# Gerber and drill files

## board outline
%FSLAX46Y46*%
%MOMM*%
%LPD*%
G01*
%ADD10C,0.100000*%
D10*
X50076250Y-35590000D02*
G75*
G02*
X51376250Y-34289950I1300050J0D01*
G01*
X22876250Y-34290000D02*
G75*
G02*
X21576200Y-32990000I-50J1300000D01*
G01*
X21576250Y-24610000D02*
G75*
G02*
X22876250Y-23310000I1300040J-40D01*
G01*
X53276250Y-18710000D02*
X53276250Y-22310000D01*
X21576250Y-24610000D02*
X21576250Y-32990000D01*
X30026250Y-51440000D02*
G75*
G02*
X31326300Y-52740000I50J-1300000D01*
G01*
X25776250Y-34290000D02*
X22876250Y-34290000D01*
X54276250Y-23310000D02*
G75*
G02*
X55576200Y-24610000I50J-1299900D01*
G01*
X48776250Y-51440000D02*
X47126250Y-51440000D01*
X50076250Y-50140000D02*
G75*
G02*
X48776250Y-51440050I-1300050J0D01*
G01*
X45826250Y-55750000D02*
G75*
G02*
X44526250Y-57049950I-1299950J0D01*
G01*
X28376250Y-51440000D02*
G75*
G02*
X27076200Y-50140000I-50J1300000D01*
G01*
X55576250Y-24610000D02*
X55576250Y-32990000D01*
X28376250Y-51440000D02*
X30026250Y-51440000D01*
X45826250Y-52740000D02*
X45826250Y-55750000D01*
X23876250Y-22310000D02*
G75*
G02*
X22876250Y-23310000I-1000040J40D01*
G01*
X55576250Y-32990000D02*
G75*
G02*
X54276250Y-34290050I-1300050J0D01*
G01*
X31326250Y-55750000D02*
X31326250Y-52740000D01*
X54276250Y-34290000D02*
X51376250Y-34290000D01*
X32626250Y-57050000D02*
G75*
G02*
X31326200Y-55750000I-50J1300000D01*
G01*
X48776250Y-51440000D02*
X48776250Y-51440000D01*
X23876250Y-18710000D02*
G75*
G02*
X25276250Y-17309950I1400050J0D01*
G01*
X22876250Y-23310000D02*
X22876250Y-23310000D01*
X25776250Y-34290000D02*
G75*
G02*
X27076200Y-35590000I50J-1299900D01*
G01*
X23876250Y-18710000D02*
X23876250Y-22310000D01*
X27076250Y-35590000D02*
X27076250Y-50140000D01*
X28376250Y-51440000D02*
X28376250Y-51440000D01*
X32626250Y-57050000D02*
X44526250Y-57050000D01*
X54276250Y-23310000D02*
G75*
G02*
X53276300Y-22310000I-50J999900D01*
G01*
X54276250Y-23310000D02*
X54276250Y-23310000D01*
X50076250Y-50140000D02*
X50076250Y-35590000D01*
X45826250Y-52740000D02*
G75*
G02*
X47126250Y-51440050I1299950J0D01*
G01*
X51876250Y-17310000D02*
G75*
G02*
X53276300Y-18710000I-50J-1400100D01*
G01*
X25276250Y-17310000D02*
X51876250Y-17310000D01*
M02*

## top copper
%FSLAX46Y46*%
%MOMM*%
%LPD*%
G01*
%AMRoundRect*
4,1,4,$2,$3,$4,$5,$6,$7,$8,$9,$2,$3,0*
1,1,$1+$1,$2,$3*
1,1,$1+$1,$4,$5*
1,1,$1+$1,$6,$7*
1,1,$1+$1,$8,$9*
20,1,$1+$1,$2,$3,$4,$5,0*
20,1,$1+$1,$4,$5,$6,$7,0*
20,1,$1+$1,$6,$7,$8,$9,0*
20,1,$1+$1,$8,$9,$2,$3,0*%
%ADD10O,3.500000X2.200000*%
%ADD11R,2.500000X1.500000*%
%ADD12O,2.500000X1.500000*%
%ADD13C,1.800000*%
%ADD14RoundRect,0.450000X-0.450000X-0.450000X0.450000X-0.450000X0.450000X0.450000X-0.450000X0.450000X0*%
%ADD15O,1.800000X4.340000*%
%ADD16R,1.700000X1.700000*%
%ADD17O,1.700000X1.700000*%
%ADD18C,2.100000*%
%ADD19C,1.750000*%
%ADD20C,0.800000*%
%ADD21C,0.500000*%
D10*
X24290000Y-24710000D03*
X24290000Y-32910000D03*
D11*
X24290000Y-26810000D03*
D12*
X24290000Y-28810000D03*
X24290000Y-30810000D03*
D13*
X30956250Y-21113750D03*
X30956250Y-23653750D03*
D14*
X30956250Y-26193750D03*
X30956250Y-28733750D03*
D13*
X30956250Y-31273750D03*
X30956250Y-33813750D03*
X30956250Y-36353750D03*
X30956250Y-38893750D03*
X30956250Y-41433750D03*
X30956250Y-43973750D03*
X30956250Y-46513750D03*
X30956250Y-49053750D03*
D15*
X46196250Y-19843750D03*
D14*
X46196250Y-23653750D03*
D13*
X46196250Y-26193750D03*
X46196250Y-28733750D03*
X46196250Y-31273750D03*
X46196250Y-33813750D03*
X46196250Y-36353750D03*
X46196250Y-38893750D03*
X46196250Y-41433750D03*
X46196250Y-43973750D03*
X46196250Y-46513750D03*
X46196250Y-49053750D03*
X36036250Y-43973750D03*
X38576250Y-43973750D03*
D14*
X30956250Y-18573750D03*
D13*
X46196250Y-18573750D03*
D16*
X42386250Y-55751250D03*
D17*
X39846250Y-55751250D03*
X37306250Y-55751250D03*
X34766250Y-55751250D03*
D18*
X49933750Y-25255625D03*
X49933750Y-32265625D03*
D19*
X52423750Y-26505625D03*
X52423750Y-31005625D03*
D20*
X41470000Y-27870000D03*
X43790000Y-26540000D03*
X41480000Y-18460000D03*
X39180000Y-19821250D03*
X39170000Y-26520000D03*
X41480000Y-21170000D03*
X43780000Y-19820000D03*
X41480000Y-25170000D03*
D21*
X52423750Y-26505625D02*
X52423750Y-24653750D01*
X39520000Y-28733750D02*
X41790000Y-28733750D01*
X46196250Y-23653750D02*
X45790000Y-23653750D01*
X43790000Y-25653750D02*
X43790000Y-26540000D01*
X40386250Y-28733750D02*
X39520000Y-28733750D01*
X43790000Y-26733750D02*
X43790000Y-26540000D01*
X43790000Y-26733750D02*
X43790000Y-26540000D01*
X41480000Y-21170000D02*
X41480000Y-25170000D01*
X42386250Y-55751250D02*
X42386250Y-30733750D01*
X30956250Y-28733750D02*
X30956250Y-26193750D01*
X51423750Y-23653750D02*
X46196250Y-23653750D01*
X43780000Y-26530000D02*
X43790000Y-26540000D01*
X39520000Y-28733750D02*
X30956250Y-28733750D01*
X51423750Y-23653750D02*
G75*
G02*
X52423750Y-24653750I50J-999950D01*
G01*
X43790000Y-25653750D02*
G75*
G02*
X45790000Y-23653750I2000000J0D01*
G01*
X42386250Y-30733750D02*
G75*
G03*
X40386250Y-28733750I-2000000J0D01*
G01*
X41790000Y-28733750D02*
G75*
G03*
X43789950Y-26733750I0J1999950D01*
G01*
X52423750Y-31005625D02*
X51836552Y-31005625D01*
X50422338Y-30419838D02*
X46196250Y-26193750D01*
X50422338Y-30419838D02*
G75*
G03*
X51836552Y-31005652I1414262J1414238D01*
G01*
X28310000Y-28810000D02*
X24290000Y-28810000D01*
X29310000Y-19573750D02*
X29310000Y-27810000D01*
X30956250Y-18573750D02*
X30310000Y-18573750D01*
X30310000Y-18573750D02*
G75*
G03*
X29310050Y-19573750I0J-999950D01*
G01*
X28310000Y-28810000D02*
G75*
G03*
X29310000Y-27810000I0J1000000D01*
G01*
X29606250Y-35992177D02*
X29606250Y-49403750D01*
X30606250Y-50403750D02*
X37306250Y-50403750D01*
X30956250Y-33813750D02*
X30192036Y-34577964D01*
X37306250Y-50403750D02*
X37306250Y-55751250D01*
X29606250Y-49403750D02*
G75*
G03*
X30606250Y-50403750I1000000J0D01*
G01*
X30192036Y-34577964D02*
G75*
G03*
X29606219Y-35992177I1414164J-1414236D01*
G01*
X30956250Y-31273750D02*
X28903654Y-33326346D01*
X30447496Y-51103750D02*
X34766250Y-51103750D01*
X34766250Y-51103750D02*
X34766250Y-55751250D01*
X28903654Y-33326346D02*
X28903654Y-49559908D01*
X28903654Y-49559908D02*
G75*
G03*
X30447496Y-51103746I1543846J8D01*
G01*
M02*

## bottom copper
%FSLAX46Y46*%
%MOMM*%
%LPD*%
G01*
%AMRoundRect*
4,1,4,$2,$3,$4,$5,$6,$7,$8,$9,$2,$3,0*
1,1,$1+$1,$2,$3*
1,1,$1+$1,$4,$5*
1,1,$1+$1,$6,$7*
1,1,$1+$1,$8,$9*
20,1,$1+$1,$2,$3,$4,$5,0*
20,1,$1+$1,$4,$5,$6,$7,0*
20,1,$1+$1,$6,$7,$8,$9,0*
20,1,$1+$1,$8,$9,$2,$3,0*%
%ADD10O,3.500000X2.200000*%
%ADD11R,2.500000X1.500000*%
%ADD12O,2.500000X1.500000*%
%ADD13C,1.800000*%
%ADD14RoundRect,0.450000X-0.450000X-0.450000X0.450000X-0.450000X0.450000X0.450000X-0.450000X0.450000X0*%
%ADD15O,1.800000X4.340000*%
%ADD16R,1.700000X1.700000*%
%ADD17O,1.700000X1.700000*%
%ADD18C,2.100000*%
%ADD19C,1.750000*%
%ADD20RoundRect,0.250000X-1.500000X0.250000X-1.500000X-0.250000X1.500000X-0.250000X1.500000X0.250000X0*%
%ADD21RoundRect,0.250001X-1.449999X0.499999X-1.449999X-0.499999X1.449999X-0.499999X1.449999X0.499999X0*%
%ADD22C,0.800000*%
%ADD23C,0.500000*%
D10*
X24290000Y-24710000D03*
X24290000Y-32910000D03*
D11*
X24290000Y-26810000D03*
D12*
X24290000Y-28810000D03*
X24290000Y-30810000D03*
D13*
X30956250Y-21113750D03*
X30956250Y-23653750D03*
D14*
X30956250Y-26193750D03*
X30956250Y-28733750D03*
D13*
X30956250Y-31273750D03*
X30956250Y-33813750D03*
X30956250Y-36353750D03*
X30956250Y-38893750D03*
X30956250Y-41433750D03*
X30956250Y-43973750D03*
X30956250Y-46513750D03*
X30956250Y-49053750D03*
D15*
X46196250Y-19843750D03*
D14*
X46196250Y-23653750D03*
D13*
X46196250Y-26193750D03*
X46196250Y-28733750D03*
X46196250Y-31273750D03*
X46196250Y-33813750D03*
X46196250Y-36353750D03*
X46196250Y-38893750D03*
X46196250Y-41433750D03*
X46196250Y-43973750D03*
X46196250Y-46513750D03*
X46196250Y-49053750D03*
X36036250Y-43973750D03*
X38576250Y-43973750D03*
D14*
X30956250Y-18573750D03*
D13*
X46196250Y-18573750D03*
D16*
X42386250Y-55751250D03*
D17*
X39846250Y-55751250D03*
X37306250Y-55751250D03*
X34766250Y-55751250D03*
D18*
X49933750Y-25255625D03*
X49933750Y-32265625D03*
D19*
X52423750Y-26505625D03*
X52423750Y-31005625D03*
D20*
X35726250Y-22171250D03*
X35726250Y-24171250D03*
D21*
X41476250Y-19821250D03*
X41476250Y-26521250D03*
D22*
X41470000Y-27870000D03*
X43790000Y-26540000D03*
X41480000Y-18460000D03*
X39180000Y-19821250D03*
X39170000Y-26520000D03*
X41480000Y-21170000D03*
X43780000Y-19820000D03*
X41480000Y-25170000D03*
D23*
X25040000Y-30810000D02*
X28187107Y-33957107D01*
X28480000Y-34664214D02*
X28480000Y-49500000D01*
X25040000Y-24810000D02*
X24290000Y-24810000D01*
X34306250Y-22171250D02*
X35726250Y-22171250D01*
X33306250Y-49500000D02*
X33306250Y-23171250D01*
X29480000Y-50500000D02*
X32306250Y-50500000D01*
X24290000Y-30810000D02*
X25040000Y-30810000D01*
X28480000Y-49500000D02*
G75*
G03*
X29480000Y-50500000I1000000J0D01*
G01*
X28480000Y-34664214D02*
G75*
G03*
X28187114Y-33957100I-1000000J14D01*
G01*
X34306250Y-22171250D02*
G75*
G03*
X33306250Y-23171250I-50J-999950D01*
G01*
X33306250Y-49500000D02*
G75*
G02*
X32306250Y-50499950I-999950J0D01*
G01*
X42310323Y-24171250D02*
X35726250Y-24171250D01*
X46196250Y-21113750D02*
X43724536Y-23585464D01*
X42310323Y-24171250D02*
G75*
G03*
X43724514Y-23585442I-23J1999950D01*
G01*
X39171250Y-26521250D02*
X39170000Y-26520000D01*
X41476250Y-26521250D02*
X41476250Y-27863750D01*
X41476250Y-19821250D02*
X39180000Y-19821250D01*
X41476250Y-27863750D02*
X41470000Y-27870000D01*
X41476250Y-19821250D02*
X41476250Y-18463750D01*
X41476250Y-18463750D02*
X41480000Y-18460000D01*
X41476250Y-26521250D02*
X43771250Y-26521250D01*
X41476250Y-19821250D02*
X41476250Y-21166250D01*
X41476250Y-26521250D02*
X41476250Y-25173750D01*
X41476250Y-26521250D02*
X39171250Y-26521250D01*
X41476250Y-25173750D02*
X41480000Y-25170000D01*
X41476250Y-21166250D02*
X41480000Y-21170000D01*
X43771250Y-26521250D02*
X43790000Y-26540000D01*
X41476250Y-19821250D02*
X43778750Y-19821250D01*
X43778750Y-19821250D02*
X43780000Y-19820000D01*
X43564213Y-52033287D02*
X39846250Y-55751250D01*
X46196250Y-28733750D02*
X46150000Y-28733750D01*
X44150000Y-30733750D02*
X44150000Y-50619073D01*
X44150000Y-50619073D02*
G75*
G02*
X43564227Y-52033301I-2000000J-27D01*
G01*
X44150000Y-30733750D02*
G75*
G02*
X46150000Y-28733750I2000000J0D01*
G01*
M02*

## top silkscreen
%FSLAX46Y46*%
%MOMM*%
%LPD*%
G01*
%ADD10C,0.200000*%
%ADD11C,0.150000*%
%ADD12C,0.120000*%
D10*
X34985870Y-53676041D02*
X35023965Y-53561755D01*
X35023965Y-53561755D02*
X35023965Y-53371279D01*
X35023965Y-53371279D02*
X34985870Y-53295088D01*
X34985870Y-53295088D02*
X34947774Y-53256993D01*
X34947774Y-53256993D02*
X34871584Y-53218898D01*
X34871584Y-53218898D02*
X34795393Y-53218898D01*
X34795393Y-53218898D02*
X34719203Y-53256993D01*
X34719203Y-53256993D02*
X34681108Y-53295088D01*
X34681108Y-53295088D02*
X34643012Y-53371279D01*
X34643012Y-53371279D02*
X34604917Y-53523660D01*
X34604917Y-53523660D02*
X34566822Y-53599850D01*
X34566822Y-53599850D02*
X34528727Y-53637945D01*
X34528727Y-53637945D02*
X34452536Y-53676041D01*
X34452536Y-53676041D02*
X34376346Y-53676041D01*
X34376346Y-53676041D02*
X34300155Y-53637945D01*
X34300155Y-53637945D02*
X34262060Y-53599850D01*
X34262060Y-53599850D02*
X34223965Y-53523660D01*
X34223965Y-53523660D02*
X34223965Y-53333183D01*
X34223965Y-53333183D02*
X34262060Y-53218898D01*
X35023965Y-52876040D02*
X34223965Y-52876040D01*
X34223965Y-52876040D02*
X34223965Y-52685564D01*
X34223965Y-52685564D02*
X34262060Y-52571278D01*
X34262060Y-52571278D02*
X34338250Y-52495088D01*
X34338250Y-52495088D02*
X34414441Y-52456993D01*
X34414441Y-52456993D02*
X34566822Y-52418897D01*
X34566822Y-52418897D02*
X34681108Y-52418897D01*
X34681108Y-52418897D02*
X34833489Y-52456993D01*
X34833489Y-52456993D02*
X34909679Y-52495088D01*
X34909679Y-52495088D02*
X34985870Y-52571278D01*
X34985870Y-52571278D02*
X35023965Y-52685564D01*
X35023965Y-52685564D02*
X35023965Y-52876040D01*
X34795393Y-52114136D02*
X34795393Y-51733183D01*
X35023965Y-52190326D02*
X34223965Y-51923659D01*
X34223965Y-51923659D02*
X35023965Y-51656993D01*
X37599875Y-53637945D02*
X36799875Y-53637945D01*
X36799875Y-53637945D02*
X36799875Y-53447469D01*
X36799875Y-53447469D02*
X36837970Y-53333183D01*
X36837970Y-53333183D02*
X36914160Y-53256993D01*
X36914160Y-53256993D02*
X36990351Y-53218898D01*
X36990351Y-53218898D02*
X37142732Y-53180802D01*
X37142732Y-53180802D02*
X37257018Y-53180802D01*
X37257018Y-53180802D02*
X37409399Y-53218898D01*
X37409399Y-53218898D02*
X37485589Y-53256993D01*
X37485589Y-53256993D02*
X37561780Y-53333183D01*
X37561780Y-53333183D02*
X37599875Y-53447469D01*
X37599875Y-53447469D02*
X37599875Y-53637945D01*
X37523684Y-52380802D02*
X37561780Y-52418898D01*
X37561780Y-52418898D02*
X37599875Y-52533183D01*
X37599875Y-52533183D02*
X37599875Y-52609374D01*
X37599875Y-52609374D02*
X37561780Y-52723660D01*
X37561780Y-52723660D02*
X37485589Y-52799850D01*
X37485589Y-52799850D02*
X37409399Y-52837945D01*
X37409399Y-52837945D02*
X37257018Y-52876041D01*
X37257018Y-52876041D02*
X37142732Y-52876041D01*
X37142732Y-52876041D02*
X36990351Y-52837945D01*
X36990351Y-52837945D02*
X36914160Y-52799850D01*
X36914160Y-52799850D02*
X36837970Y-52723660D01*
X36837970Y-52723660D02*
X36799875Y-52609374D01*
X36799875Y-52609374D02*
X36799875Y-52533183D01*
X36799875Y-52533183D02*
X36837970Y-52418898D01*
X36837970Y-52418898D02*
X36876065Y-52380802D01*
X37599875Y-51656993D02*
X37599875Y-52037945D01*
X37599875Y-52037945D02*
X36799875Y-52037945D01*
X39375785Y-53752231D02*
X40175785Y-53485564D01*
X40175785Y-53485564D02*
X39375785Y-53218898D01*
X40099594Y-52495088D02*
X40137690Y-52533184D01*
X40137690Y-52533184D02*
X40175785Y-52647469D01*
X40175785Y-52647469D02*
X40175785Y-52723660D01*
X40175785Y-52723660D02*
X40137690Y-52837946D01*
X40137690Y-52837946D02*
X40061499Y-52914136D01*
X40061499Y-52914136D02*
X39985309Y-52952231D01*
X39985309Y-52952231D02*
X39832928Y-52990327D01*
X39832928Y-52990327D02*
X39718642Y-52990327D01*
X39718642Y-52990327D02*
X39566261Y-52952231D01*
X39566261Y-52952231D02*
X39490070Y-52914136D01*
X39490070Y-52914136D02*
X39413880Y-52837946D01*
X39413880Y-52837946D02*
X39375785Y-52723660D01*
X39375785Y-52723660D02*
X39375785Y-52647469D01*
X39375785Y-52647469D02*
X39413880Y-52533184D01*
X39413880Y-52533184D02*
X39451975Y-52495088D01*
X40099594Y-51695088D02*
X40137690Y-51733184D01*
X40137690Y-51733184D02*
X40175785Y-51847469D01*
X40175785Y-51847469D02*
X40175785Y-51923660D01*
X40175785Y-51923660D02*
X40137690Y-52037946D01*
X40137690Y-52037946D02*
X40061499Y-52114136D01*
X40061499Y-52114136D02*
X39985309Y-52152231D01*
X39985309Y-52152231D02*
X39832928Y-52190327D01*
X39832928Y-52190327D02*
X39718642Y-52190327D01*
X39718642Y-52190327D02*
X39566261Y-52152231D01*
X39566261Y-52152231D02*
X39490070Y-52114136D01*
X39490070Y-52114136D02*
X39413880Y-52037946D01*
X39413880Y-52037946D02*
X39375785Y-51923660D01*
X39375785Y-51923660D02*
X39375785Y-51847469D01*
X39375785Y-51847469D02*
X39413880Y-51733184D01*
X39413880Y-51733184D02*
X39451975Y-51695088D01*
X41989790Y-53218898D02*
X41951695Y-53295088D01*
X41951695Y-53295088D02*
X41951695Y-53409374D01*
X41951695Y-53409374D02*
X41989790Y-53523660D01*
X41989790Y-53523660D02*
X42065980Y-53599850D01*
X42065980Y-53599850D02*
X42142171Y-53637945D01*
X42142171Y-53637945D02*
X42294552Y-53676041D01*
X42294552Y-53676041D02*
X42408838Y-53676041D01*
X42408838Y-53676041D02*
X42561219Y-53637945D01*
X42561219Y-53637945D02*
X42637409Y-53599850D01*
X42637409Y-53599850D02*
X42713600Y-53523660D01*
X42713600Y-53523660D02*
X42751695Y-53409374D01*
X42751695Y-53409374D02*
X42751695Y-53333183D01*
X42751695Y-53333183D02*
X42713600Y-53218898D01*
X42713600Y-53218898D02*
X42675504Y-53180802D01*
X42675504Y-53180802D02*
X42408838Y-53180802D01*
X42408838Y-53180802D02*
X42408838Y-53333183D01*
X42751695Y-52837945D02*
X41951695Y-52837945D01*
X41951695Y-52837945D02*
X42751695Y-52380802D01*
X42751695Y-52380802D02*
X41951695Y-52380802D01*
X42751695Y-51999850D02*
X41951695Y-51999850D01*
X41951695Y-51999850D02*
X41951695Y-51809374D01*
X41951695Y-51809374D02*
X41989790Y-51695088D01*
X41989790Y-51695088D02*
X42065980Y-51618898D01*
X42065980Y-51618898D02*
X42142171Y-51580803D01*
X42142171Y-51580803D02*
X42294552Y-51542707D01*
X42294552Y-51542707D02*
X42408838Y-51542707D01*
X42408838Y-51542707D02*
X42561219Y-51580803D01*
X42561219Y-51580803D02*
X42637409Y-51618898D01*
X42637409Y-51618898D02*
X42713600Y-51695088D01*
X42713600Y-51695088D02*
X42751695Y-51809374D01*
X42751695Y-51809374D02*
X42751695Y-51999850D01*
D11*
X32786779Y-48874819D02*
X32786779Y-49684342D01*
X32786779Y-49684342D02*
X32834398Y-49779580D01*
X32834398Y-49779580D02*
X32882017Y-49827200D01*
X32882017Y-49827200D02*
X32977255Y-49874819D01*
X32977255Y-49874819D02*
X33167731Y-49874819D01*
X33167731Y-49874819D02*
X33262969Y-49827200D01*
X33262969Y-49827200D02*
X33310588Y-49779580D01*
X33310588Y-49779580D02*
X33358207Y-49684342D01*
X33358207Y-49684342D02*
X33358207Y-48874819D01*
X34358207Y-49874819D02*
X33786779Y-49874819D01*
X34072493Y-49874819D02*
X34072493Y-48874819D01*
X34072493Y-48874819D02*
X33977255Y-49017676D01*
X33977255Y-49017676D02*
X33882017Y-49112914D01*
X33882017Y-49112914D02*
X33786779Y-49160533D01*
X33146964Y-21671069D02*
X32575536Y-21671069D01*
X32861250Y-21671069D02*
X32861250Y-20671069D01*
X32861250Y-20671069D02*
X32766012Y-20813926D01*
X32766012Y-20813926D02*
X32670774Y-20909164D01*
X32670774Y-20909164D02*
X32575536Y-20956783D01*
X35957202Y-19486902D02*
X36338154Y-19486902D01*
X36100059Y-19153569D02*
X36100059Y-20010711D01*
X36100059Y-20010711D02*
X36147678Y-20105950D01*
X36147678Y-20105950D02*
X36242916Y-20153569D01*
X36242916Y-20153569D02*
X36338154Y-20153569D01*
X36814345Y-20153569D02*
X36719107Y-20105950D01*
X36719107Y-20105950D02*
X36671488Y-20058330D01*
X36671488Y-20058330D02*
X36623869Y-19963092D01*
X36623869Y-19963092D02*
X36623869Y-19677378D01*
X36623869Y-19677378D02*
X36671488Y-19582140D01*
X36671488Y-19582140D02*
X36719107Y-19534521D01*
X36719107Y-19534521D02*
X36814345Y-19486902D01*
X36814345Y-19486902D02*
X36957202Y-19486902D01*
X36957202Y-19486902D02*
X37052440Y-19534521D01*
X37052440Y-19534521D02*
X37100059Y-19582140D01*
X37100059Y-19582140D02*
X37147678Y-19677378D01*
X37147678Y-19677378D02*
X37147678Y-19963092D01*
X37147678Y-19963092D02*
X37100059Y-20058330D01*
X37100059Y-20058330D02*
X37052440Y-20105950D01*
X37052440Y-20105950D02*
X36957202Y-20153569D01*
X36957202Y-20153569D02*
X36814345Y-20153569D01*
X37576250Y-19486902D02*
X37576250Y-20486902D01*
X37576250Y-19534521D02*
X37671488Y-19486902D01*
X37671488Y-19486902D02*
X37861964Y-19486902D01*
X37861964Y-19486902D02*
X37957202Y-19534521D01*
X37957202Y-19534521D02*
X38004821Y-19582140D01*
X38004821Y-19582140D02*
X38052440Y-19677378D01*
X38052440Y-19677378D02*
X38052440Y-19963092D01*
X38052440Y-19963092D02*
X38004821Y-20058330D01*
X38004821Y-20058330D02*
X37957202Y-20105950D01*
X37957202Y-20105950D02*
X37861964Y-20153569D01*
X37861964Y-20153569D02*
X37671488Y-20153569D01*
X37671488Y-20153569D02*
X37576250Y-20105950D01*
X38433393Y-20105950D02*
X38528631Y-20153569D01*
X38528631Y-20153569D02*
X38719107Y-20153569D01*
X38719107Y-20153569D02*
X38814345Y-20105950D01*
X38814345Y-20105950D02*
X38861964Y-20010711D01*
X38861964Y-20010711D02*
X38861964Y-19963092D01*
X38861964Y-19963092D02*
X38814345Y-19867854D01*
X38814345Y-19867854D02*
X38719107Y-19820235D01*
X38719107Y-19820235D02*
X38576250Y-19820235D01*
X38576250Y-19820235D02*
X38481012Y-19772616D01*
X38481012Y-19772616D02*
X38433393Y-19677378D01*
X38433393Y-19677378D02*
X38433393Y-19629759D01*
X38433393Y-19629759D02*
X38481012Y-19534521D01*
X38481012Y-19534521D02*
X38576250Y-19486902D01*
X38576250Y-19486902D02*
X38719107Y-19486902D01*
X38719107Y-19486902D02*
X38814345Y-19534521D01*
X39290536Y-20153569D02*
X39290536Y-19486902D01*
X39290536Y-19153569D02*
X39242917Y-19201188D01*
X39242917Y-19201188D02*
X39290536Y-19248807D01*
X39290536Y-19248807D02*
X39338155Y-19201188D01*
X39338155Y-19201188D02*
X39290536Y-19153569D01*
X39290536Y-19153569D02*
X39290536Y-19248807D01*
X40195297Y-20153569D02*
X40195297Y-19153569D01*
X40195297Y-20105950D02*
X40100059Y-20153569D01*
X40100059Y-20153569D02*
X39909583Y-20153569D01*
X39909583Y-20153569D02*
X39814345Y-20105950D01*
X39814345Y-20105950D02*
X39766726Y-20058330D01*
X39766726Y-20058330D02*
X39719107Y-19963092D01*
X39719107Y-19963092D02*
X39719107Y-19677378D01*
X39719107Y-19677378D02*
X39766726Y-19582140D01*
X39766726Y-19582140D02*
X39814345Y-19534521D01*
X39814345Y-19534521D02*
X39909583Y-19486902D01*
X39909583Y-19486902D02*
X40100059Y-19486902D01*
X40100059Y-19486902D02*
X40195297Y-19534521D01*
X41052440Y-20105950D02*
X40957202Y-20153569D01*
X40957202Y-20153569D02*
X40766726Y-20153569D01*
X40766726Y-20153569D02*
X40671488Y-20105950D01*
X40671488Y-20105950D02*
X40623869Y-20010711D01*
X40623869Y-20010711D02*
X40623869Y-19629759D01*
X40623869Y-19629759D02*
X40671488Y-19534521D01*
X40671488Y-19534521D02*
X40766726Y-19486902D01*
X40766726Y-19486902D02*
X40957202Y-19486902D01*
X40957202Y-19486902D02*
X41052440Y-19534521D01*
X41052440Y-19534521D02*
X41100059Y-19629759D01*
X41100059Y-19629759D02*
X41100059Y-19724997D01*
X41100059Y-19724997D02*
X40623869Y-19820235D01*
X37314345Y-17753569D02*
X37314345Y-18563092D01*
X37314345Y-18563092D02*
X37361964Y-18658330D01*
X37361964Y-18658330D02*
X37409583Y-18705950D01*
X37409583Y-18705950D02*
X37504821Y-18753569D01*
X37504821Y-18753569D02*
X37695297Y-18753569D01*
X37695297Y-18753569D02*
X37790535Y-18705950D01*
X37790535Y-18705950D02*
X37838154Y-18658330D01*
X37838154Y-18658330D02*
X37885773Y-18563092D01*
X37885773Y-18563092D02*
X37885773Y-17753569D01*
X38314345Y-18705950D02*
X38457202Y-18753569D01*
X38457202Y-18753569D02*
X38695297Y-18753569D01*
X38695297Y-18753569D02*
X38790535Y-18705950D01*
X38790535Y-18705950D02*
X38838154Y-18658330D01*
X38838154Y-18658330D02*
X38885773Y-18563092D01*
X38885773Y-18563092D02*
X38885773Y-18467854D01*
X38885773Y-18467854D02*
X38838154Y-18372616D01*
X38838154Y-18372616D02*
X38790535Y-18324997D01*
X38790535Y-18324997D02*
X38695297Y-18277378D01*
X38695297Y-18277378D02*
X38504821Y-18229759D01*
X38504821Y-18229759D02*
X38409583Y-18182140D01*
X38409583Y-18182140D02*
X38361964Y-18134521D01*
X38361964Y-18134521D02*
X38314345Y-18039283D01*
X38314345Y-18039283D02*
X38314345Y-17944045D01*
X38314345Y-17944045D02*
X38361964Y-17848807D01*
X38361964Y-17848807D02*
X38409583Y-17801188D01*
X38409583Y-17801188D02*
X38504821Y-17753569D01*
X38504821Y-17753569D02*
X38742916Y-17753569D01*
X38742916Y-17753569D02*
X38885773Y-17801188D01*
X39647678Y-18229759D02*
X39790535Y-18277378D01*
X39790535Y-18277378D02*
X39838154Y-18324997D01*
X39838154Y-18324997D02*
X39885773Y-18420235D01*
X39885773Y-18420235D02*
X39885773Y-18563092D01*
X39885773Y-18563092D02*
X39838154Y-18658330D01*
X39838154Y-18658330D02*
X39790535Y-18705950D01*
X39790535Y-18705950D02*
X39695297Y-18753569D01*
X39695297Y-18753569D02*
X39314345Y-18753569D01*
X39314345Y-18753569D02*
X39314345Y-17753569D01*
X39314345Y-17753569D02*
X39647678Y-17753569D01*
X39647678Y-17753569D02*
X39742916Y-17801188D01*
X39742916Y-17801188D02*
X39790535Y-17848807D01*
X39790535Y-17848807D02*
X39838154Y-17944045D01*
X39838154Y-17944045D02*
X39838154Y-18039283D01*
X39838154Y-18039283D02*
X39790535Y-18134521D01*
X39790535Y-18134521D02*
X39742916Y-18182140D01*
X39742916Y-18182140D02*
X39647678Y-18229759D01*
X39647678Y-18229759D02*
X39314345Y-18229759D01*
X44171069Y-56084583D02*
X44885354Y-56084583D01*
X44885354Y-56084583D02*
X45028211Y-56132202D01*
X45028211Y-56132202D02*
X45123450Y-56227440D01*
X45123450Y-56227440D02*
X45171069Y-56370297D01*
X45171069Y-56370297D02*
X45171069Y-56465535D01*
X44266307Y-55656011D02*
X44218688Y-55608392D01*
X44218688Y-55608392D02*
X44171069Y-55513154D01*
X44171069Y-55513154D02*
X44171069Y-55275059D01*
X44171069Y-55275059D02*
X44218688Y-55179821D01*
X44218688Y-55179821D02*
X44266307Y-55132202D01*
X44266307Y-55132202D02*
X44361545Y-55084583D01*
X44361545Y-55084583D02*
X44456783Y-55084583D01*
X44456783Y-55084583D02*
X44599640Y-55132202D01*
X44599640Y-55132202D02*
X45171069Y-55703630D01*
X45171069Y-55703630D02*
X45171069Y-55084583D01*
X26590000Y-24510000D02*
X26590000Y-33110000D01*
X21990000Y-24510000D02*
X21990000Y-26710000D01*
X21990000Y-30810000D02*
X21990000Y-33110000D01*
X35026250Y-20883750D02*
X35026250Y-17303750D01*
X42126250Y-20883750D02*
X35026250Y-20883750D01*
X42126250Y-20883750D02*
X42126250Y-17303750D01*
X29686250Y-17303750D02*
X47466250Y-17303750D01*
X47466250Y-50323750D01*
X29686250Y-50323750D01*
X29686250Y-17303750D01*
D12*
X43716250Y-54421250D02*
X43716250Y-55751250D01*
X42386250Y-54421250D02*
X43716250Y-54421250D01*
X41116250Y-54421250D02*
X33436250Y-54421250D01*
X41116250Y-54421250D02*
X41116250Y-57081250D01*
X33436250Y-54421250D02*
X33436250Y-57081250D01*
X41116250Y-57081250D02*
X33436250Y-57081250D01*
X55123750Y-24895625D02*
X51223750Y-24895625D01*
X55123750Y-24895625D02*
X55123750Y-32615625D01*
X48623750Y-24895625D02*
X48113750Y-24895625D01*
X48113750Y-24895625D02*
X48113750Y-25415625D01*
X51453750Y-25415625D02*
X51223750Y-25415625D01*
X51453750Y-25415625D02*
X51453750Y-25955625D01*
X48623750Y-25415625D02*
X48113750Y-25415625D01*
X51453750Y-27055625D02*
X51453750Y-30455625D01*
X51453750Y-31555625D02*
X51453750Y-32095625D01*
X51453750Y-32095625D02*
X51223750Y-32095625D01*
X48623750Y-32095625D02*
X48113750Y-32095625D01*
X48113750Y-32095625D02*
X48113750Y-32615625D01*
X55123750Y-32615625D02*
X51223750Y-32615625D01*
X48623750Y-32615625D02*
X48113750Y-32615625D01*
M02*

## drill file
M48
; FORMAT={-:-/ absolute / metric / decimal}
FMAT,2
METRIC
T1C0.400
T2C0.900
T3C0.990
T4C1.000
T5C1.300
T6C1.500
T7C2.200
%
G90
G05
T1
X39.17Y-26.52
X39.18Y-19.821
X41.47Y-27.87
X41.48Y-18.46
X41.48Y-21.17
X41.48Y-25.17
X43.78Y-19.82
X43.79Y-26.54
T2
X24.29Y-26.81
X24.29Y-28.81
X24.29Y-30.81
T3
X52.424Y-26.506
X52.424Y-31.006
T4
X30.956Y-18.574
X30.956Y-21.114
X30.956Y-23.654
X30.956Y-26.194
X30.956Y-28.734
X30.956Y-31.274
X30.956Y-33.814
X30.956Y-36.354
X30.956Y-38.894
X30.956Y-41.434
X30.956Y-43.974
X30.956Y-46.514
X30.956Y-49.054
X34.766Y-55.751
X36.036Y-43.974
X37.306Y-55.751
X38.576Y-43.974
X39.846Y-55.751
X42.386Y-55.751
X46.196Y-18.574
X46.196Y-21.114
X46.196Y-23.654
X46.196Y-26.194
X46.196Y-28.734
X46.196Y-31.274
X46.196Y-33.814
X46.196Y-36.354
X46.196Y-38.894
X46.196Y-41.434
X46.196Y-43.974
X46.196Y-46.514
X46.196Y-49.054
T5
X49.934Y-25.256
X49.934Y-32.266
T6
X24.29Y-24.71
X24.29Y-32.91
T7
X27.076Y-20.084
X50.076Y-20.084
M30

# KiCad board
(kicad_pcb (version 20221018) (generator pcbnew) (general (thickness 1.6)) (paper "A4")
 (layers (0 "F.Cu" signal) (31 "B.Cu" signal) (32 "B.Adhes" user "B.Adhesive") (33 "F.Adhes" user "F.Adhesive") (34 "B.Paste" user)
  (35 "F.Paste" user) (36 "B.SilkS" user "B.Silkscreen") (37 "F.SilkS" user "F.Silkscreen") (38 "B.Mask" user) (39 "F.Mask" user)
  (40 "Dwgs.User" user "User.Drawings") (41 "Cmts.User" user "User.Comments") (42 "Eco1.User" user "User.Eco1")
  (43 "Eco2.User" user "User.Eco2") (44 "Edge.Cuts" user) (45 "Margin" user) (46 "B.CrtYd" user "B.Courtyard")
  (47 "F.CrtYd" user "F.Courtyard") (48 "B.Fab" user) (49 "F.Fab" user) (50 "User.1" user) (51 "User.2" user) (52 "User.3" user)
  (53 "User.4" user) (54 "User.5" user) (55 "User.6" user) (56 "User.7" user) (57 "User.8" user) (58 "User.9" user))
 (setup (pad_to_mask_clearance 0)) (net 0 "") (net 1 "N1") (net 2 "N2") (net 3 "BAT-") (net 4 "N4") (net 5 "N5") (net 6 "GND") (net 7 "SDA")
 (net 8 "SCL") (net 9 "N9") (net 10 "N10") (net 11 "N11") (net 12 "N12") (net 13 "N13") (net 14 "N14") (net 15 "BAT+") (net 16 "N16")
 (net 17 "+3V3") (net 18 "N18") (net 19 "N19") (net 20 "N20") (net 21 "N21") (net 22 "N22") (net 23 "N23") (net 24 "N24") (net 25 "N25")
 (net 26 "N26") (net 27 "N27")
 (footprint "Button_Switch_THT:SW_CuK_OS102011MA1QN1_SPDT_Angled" (layer "F.Cu") (at 24.29 26.81 -90)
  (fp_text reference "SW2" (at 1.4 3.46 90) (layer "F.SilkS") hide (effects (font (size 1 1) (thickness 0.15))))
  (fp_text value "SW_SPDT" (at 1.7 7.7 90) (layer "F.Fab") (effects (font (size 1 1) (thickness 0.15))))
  (fp_line (start -2.3 -2.3) (end 6.3 -2.3) (stroke (width 0.15) (type solid)) (layer "F.SilkS"))
  (fp_line (start -2.3 2.3) (end -0.1 2.3) (stroke (width 0.15) (type solid)) (layer "F.SilkS"))
  (fp_line (start 4 2.3) (end 6.3 2.3) (stroke (width 0.15) (type solid)) (layer "F.SilkS"))
  (pad "" thru_hole oval (at -2.1 0 270) (size 2.2 3.5) (drill 1.5) (layers "*.Cu" "*.Mask"))
  (pad "" thru_hole oval (at 6.1 0 270) (size 2.2 3.5) (drill 1.5) (layers "*.Cu" "*.Mask"))
  (pad "1" thru_hole rect (at 0 0 270) (size 1.5 2.5) (drill 0.9) (layers "*.Cu" "*.Mask") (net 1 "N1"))
  (pad "2" thru_hole oval (at 2 0 270) (size 1.5 2.5) (drill 0.9) (layers "*.Cu" "*.Mask") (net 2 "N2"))
  (pad "3" thru_hole oval (at 4 0 270) (size 1.5 2.5) (drill 0.9) (layers "*.Cu" "*.Mask") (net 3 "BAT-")))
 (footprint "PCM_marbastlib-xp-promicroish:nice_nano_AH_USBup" (layer "F.Cu") (at 38.57625 35.08375)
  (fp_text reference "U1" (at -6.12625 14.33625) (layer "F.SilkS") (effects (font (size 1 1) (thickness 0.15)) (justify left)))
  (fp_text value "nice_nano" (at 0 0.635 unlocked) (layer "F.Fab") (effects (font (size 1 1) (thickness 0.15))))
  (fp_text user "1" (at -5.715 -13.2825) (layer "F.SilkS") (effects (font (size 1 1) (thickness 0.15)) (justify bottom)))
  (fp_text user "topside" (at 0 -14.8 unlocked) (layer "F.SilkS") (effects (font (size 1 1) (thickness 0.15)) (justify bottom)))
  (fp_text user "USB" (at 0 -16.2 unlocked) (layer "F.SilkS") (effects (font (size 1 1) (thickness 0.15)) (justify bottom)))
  (fp_line (start -3.55 -14.2) (end -3.55 -17.78) (stroke (width 0.15) (type default)) (layer "F.SilkS"))
  (fp_line (start 3.55 -14.2) (end -3.55 -14.2) (stroke (width 0.15) (type default)) (layer "F.SilkS"))
  (fp_line (start 3.55 -14.2) (end 3.55 -17.78) (stroke (width 0.15) (type default)) (layer "F.SilkS"))
  (fp_rect (start -8.89 -17.78) (end 8.89 15.24) (stroke (width 0.15) (type solid)) (fill none) (layer "F.SilkS"))
  (pad "1" thru_hole circle (at -7.62 -13.97) (size 1.8 1.8) (drill 1) (layers "*.Cu" "B.Mask") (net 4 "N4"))
  (pad "2" thru_hole circle (at -7.62 -11.43) (size 1.8 1.8) (drill 1) (layers "*.Cu" "B.Mask") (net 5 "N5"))
  (pad "3" thru_hole roundrect (at -7.62 -8.89) (size 1.8 1.8) (drill 1) (layers "*.Cu" "B.Mask") (roundrect_rratio 0.25) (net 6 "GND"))
  (pad "4" thru_hole roundrect (at -7.62 -6.35) (size 1.8 1.8) (drill 1) (layers "*.Cu" "B.Mask") (roundrect_rratio 0.25) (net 6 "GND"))
  (pad "5" thru_hole circle (at -7.62 -3.81) (size 1.8 1.8) (drill 1) (layers "*.Cu" "B.Mask") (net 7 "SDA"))
  (pad "6" thru_hole circle (at -7.62 -1.27) (size 1.8 1.8) (drill 1) (layers "*.Cu" "B.Mask") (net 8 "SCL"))
  (pad "7" thru_hole circle (at -7.62 1.27) (size 1.8 1.8) (drill 1) (layers "*.Cu" "B.Mask") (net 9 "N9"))
  (pad "8" thru_hole circle (at -7.62 3.81) (size 1.8 1.8) (drill 1) (layers "*.Cu" "B.Mask") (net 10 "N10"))
  (pad "9" thru_hole circle (at -7.62 6.35) (size 1.8 1.8) (drill 1) (layers "*.Cu" "B.Mask") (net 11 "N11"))
  (pad "10" thru_hole circle (at -7.62 8.89) (size 1.8 1.8) (drill 1) (layers "*.Cu" "B.Mask") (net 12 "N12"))
  (pad "11" thru_hole circle (at -7.62 11.43) (size 1.8 1.8) (drill 1) (layers "*.Cu" "B.Mask") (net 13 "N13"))
  (pad "12" thru_hole circle (at -7.62 13.97) (size 1.8 1.8) (drill 1) (layers "*.Cu" "B.Mask") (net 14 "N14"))
  (pad "13" thru_hole oval (at 7.62 -13.97) (size 1.8 4.34) (drill 1 (offset 0 -1.27)) (layers "*.Cu" "B.Mask") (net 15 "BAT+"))
  (pad "14" thru_hole roundrect (at 7.62 -11.43) (size 1.8 1.8) (drill 1) (layers "*.Cu" "B.Mask") (roundrect_rratio 0.25) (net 6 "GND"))
  (pad "15" thru_hole circle (at 7.62 -8.89) (size 1.8 1.8) (drill 1) (layers "*.Cu" "B.Mask") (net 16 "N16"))
  (pad "16" thru_hole circle (at 7.62 -6.35) (size 1.8 1.8) (drill 1) (layers "*.Cu" "B.Mask") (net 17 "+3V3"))
  (pad "17" thru_hole circle (at 7.62 -3.81) (size 1.8 1.8) (drill 1) (layers "*.Cu" "B.Mask") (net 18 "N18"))
  (pad "18" thru_hole circle (at 7.62 -1.27) (size 1.8 1.8) (drill 1) (layers "*.Cu" "B.Mask") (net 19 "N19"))
  (pad "19" thru_hole circle (at 7.62 1.27) (size 1.8 1.8) (drill 1) (layers "*.Cu" "B.Mask") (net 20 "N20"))
  (pad "20" thru_hole circle (at 7.62 3.81) (size 1.8 1.8) (drill 1) (layers "*.Cu" "B.Mask") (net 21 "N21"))
  (pad "21" thru_hole circle (at 7.62 6.35) (size 1.8 1.8) (drill 1) (layers "*.Cu" "B.Mask") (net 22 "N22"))
  (pad "22" thru_hole circle (at 7.62 8.89) (size 1.8 1.8) (drill 1) (layers "*.Cu" "B.Mask") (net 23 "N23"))
  (pad "23" thru_hole circle (at 7.62 11.43) (size 1.8 1.8) (drill 1) (layers "*.Cu" "B.Mask") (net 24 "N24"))
  (pad "24" thru_hole circle (at 7.62 13.97) (size 1.8 1.8) (drill 1) (layers "*.Cu" "B.Mask") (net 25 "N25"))
  (pad "26" thru_hole circle (at -2.54 8.89) (size 1.8 1.8) (drill 1) (layers "*.Cu" "B.Mask") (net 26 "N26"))
  (pad "27" thru_hole circle (at 0 8.89) (size 1.8 1.8) (drill 1) (layers "*.Cu" "B.Mask") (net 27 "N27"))
  (pad "28" thru_hole roundrect (at -7.62 -16.51) (size 1.8 1.8) (drill 1) (layers "*.Cu" "B.Mask") (roundrect_rratio 0.25) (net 2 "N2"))
  (pad "29" thru_hole circle (at 7.62 -16.51) (size 1.8 1.8) (drill 1) (layers "*.Cu" "B.Mask") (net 15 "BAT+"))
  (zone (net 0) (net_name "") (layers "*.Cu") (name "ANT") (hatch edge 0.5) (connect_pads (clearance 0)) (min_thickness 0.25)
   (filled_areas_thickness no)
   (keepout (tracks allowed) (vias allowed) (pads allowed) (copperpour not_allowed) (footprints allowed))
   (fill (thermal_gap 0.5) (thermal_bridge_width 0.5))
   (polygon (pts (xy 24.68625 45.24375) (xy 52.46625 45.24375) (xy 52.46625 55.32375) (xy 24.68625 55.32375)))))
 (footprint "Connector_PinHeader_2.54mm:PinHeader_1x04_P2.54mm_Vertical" (layer "F.Cu") (at 42.38625 55.75125 -90)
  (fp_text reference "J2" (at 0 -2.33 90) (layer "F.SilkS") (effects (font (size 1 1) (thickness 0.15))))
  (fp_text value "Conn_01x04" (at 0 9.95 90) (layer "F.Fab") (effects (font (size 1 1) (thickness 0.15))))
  (fp_line (start -1.33 -1.33) (end 0 -1.33) (stroke (width 0.12) (type solid)) (layer "F.SilkS"))
  (fp_line (start -1.33 0) (end -1.33 -1.33) (stroke (width 0.12) (type solid)) (layer "F.SilkS"))
  (fp_line (start -1.33 1.27) (end -1.33 8.95) (stroke (width 0.12) (type solid)) (layer "F.SilkS"))
  (fp_line (start -1.33 1.27) (end 1.33 1.27) (stroke (width 0.12) (type solid)) (layer "F.SilkS"))
  (fp_line (start -1.33 8.95) (end 1.33 8.95) (stroke (width 0.12) (type solid)) (layer "F.SilkS"))
  (fp_line (start 1.33 1.27) (end 1.33 8.95) (stroke (width 0.12) (type solid)) (layer "F.SilkS"))
  (pad "1" thru_hole rect (at 0 0 270) (size 1.7 1.7) (drill 1) (layers "*.Cu" "*.Mask") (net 6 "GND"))
  (pad "2" thru_hole oval (at 0 2.54 270) (size 1.7 1.7) (drill 1) (layers "*.Cu" "*.Mask") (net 17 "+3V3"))
  (pad "3" thru_hole oval (at 0 5.08 270) (size 1.7 1.7) (drill 1) (layers "*.Cu" "*.Mask") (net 8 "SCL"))
  (pad "4" thru_hole oval (at 0 7.62 270) (size 1.7 1.7) (drill 1) (layers "*.Cu" "*.Mask") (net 7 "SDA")))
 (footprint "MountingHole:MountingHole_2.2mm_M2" (layer "F.Cu") (at 50.07625 20.08375)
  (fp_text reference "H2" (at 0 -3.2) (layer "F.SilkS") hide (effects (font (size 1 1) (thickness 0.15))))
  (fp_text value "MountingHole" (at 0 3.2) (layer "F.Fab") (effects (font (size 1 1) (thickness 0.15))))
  (pad "" np_thru_hole circle (at 0 0) (size 2.2 2.2) (drill 2.2) (layers "*.Cu" "*.Mask")))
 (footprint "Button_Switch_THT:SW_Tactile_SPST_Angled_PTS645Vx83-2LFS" (layer "F.Cu") (at 52.42375 26.505625 -90)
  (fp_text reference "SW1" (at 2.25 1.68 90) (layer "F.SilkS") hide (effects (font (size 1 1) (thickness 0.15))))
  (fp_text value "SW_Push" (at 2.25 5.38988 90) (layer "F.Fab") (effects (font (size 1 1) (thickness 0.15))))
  (fp_line (start -1.61 -2.7) (end -1.61 1.2) (stroke (width 0.12) (type solid)) (layer "F.SilkS"))
  (fp_line (start -1.61 -2.7) (end 6.11 -2.7) (stroke (width 0.12) (type solid)) (layer "F.SilkS"))
  (fp_line (start -1.61 3.8) (end -1.61 4.31) (stroke (width 0.12) (type solid)) (layer "F.SilkS"))
  (fp_line (start -1.61 4.31) (end -1.09 4.31) (stroke (width 0.12) (type solid)) (layer "F.SilkS"))
  (fp_line (start -1.09 0.97) (end -1.09 1.2) (stroke (width 0.12) (type solid)) (layer "F.SilkS"))
  (fp_line (start -1.09 0.97) (end -0.55 0.97) (stroke (width 0.12) (type solid)) (layer "F.SilkS"))
  (fp_line (start -1.09 3.8) (end -1.09 4.31) (stroke (width 0.12) (type solid)) (layer "F.SilkS"))
  (fp_line (start 0.55 0.97) (end 3.95 0.97) (stroke (width 0.12) (type solid)) (layer "F.SilkS"))
  (fp_line (start 5.05 0.97) (end 5.59 0.97) (stroke (width 0.12) (type solid)) (layer "F.SilkS"))
  (fp_line (start 5.59 0.97) (end 5.59 1.2) (stroke (width 0.12) (type solid)) (layer "F.SilkS"))
  (fp_line (start 5.59 3.8) (end 5.59 4.31) (stroke (width 0.12) (type solid)) (layer "F.SilkS"))
  (fp_line (start 5.59 4.31) (end 6.11 4.31) (stroke (width 0.12) (type solid)) (layer "F.SilkS"))
  (fp_line (start 6.11 -2.7) (end 6.11 1.2) (stroke (width 0.12) (type solid)) (layer "F.SilkS"))
  (fp_line (start 6.11 3.8) (end 6.11 4.31) (stroke (width 0.12) (type solid)) (layer "F.SilkS"))
  (pad "" thru_hole circle (at -1.25 2.49 270) (size 2.1 2.1) (drill 1.3) (layers "*.Cu" "*.Mask"))
  (pad "" thru_hole circle (at 5.76 2.49 270) (size 2.1 2.1) (drill 1.3) (layers "*.Cu" "*.Mask"))
  (pad "1" thru_hole circle (at 0 0 270) (size 1.75 1.75) (drill 0.99) (layers "*.Cu" "*.Mask") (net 6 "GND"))
  (pad "2" thru_hole circle (at 4.5 0 270) (size 1.75 1.75) (drill 0.99) (layers "*.Cu" "*.Mask") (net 16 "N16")))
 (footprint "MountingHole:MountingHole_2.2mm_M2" (layer "F.Cu") (at 27.07625 20.08375)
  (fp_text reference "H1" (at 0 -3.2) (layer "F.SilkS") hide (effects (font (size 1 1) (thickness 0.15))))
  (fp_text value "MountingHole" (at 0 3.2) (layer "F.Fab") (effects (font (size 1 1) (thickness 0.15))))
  (pad "" np_thru_hole circle (at 0 0) (size 2.2 2.2) (drill 2.2) (layers "*.Cu" "*.Mask")))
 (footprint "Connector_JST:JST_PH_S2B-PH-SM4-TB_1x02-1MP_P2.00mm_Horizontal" (layer "B.Cu") (at 38.57625 23.17125 -90)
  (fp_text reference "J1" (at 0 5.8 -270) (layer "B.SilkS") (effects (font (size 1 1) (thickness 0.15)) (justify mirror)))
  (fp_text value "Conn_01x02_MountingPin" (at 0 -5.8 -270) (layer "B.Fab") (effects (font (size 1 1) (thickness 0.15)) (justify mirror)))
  (pad "1" smd roundrect (at -1 2.85 270) (size 1 3.5) (layers "B.Cu" "B.Paste" "B.Mask") (roundrect_rratio 0.25) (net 3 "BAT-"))
  (pad "2" smd roundrect (at 1 2.85 270) (size 1 3.5) (layers "B.Cu" "B.Paste" "B.Mask") (roundrect_rratio 0.25) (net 15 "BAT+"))
  (pad "MP" smd roundrect (at -3.35 -2.9 270) (size 1.5 3.4) (layers "B.Cu" "B.Paste" "B.Mask") (roundrect_rratio 0.1666673333)
   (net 6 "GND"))
  (pad "MP" smd roundrect (at 3.35 -2.9 270) (size 1.5 3.4) (layers "B.Cu" "B.Paste" "B.Mask") (roundrect_rratio 0.1666673333) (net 6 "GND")))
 (gr_arc (start 50.07625 35.59) (mid 50.457014 34.670779) (end 51.37625 34.29) (stroke (width 0.1) (type default)) (layer "Edge.Cuts"))
 (gr_arc (start 22.87625 34.29) (mid 21.957014 33.90925) (end 21.57625 32.99) (stroke (width 0.1) (type default)) (layer "Edge.Cuts"))
 (gr_arc (start 21.57625 24.61) (mid 21.957023 23.690773) (end 22.87625 23.31) (stroke (width 0.1) (type default)) (layer "Edge.Cuts"))
 (gr_line (start 53.27625 18.71) (end 53.27625 22.31) (stroke (width 0.1) (type default)) (layer "Edge.Cuts"))
 (gr_line (start 21.57625 24.61) (end 21.57625 32.99) (stroke (width 0.1) (type default)) (layer "Edge.Cuts"))
 (gr_arc (start 30.02625 51.44) (mid 30.945486 51.82075) (end 31.32625 52.74) (stroke (width 0.1) (type default)) (layer "Edge.Cuts"))
 (gr_line (start 25.77625 34.29) (end 22.87625 34.29) (stroke (width 0.1) (type default)) (layer "Edge.Cuts"))
 (gr_arc (start 54.27625 23.31) (mid 55.195521 23.690744) (end 55.57625 24.61) (stroke (width 0.1) (type default)) (layer "Edge.Cuts"))
 (gr_line (start 48.77625 51.44) (end 47.12625 51.44) (stroke (width 0.1) (type default)) (layer "Edge.Cuts"))
 (gr_arc (start 50.07625 50.14) (mid 49.695486 51.059221) (end 48.77625 51.44) (stroke (width 0.1) (type default)) (layer "Edge.Cuts"))
 (gr_arc (start 45.82625 55.75) (mid 45.445492 56.669256) (end 44.52625 57.05) (stroke (width 0.1) (type default)) (layer "Edge.Cuts"))
 (gr_arc (start 28.37625 51.44) (mid 27.457011 51.059239) (end 27.07625 50.14) (stroke (width 0.1) (type default)) (layer "Edge.Cuts"))
 (gr_line (start 55.57625 24.61) (end 55.57625 32.99) (stroke (width 0.1) (type default)) (layer "Edge.Cuts"))
 (gr_line (start 28.37625 51.44) (end 30.02625 51.44) (stroke (width 0.1) (type default)) (layer "Edge.Cuts"))
 (gr_line (start 45.82625 52.74) (end 45.82625 55.75) (stroke (width 0.1) (type default)) (layer "Edge.Cuts"))
 (gr_arc (start 23.87625 22.31) (mid 23.583354 23.017089) (end 22.87625 23.31) (stroke (width 0.1) (type default)) (layer "Edge.Cuts"))
 (gr_arc (start 55.57625 32.99) (mid 55.195486 33.909221) (end 54.27625 34.29) (stroke (width 0.1) (type default)) (layer "Edge.Cuts"))
 (gr_line (start 31.32625 55.75) (end 31.32625 52.74) (stroke (width 0.1) (type default)) (layer "Edge.Cuts"))
 (gr_line (start 54.27625 34.29) (end 51.37625 34.29) (stroke (width 0.1) (type default)) (layer "Edge.Cuts"))
 (gr_arc (start 32.62625 57.05) (mid 31.707014 56.66925) (end 31.32625 55.75) (stroke (width 0.1) (type default)) (layer "Edge.Cuts"))
 (gr_line (start 48.77625 51.44) (end 48.77625 51.44) (stroke (width 0.1) (type default)) (layer "Edge.Cuts"))
 (gr_arc (start 23.87625 18.71) (mid 24.286301 17.720051) (end 25.27625 17.31) (stroke (width 0.1) (type default)) (layer "Edge.Cuts"))
 (gr_line (start 22.87625 23.31) (end 22.87625 23.31) (stroke (width 0.1) (type default)) (layer "Edge.Cuts"))
 (gr_arc (start 25.77625 34.29) (mid 26.695521 34.670744) (end 27.07625 35.59) (stroke (width 0.1) (type default)) (layer "Edge.Cuts"))
 (gr_line (start 23.87625 18.71) (end 23.87625 22.31) (stroke (width 0.1) (type default)) (layer "Edge.Cuts"))
 (gr_line (start 27.07625 35.59) (end 27.07625 50.14) (stroke (width 0.1) (type default)) (layer "Edge.Cuts"))
 (gr_line (start 28.37625 51.44) (end 28.37625 51.44) (stroke (width 0.1) (type default)) (layer "Edge.Cuts"))
 (gr_line (start 32.62625 57.05) (end 44.52625 57.05) (stroke (width 0.1) (type default)) (layer "Edge.Cuts"))
 (gr_arc (start 54.27625 23.31) (mid 53.569111 23.017124) (end 53.27625 22.31) (stroke (width 0.1) (type default)) (layer "Edge.Cuts"))
 (gr_line (start 54.27625 23.31) (end 54.27625 23.31) (stroke (width 0.1) (type default)) (layer "Edge.Cuts"))
 (gr_line (start 50.07625 50.14) (end 50.07625 35.59) (stroke (width 0.1) (type default)) (layer "Edge.Cuts"))
 (gr_arc (start 45.82625 52.74) (mid 46.207008 51.820744) (end 47.12625 51.44) (stroke (width 0.1) (type default)) (layer "Edge.Cuts"))
 (gr_arc (start 51.87625 17.31) (mid 52.866167 17.720068) (end 53.27625 18.71) (stroke (width 0.1) (type default)) (layer "Edge.Cuts"))
 (gr_line (start 25.27625 17.31) (end 51.87625 17.31) (stroke (width 0.1) (type default)) (layer "Edge.Cuts"))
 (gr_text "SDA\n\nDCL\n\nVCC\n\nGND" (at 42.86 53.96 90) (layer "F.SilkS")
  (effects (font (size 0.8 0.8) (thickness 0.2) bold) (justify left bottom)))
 (segment (start 25.04 30.81) (end 28.187107 33.957107) (width 0.5) (layer "B.Cu") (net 3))
 (segment (start 28.48 34.664214) (end 28.48 49.5) (width 0.5) (layer "B.Cu") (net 3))
 (segment (start 25.04 24.81) (end 24.29 24.81) (width 0.5) (layer "B.Cu") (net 3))
 (segment (start 34.30625 22.17125) (end 35.72625 22.17125) (width 0.5) (layer "B.Cu") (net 3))
 (segment (start 33.30625 49.5) (end 33.30625 23.17125) (width 0.5) (layer "B.Cu") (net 3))
 (segment (start 29.48 50.5) (end 32.30625 50.5) (width 0.5) (layer "B.Cu") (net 3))
 (segment (start 24.29 30.81) (end 25.04 30.81) (width 0.5) (layer "B.Cu") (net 3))
 (arc (start 28.48 49.5) (mid 28.772893 50.207107) (end 29.48 50.5) (width 0.5) (layer "B.Cu") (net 3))
 (arc (start 28.48 34.664214) (mid 28.40388 34.281531) (end 28.187107 33.957107) (width 0.5) (layer "B.Cu") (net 3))
 (arc (start 34.30625 22.17125) (mid 33.599143 22.464143) (end 33.30625 23.17125) (width 0.5) (layer "B.Cu") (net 3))
 (arc (start 33.30625 49.5) (mid 33.013357 50.207107) (end 32.30625 50.5) (width 0.5) (layer "B.Cu") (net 3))
 (segment (start 42.310323 24.17125) (end 35.72625 24.17125) (width 0.5) (layer "B.Cu") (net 15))
 (segment (start 46.19625 21.11375) (end 43.724536 23.585464) (width 0.5) (layer "B.Cu") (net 15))
 (arc (start 42.310323 24.17125) (mid 43.07569 24.019009) (end 43.724536 23.585464) (width 0.5) (layer "B.Cu") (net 15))
 (segment (start 52.42375 26.505625) (end 52.42375 24.65375) (width 0.5) (layer "F.Cu") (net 6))
 (segment (start 39.52 28.73375) (end 41.79 28.73375) (width 0.5) (layer "F.Cu") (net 6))
 (segment (start 46.19625 23.65375) (end 45.79 23.65375) (width 0.5) (layer "F.Cu") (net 6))
 (segment (start 43.79 25.65375) (end 43.79 26.54) (width 0.5) (layer "F.Cu") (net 6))
 (segment (start 40.38625 28.73375) (end 39.52 28.73375) (width 0.5) (layer "F.Cu") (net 6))
 (segment (start 43.79 26.73375) (end 43.79 26.54) (width 0.5) (layer "F.Cu") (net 6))
 (segment (start 43.79 26.73375) (end 43.79 26.54) (width 0.5) (layer "F.Cu") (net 6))
 (segment (start 41.48 21.17) (end 41.48 25.17) (width 0.5) (layer "F.Cu") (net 6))
 (segment (start 42.38625 55.75125) (end 42.38625 30.73375) (width 0.5) (layer "F.Cu") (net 6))
 (segment (start 30.95625 28.73375) (end 30.95625 26.19375) (width 0.5) (layer "F.Cu") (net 6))
 (segment (start 51.42375 23.65375) (end 46.19625 23.65375) (width 0.5) (layer "F.Cu") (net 6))
 (segment (start 43.78 26.53) (end 43.79 26.54) (width 0.5) (layer "F.Cu") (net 6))
 (segment (start 39.52 28.73375) (end 30.95625 28.73375) (width 0.5) (layer "F.Cu") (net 6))
 (via (at 41.47 27.87) (size 0.8) (drill 0.4) (layers "F.Cu" "B.Cu") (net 6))
 (via (at 43.79 26.54) (size 0.8) (drill 0.4) (layers "F.Cu" "B.Cu") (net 6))
 (via (at 41.48 18.46) (size 0.8) (drill 0.4) (layers "F.Cu" "B.Cu") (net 6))
 (via (at 39.18 19.82125) (size 0.8) (drill 0.4) (layers "F.Cu" "B.Cu") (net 6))
 (via (at 39.17 26.52) (size 0.8) (drill 0.4) (layers "F.Cu" "B.Cu") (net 6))
 (via (at 41.48 21.17) (size 0.8) (drill 0.4) (layers "F.Cu" "B.Cu") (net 6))
 (via (at 43.78 19.82) (size 0.8) (drill 0.4) (layers "F.Cu" "B.Cu") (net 6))
 (via (at 41.48 25.17) (size 0.8) (drill 0.4) (layers "F.Cu" "B.Cu") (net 6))
 (arc (start 51.42375 23.65375) (mid 52.130857 23.946643) (end 52.42375 24.65375) (width 0.5) (layer "F.Cu") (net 6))
 (arc (start 43.79 25.65375) (mid 44.375786 24.239536) (end 45.79 23.65375) (width 0.5) (layer "F.Cu") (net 6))
 (arc (start 42.38625 30.73375) (mid 41.800464 29.319536) (end 40.38625 28.73375) (width 0.5) (layer "F.Cu") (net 6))
 (arc (start 41.79 28.73375) (mid 43.204214 28.147964) (end 43.79 26.73375) (width 0.5) (layer "F.Cu") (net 6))
 (segment (start 39.17125 26.52125) (end 39.17 26.52) (width 0.5) (layer "B.Cu") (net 6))
 (segment (start 41.47625 26.52125) (end 41.47625 27.86375) (width 0.5) (layer "B.Cu") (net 6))
 (segment (start 41.47625 19.82125) (end 39.18 19.82125) (width 0.5) (layer "B.Cu") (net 6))
 (segment (start 41.47625 27.86375) (end 41.47 27.87) (width 0.5) (layer "B.Cu") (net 6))
 (segment (start 41.47625 19.82125) (end 41.47625 18.46375) (width 0.5) (layer "B.Cu") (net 6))
 (segment (start 41.47625 18.46375) (end 41.48 18.46) (width 0.5) (layer "B.Cu") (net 6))
 (segment (start 41.47625 26.52125) (end 43.77125 26.52125) (width 0.5) (layer "B.Cu") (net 6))
 (segment (start 41.47625 19.82125) (end 41.47625 21.16625) (width 0.5) (layer "B.Cu") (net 6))
 (segment (start 41.47625 26.52125) (end 41.47625 25.17375) (width 0.5) (layer "B.Cu") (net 6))
 (segment (start 41.47625 26.52125) (end 39.17125 26.52125) (width 0.5) (layer "B.Cu") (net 6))
 (segment (start 41.47625 25.17375) (end 41.48 25.17) (width 0.5) (layer "B.Cu") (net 6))
 (segment (start 41.47625 21.16625) (end 41.48 21.17) (width 0.5) (layer "B.Cu") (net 6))
 (segment (start 43.77125 26.52125) (end 43.79 26.54) (width 0.5) (layer "B.Cu") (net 6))
 (segment (start 41.47625 19.82125) (end 43.77875 19.82125) (width 0.5) (layer "B.Cu") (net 6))
 (segment (start 43.77875 19.82125) (end 43.78 19.82) (width 0.5) (layer "B.Cu") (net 6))
 (segment (start 52.42375 31.005625) (end 51.836552 31.005625) (width 0.5) (layer "F.Cu") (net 16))
 (segment (start 50.422338 30.419838) (end 46.19625 26.19375) (width 0.5) (layer "F.Cu") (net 16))
 (arc (start 50.422338 30.419838) (mid 51.071185 30.853384) (end 51.836552 31.005625) (width 0.5) (layer "F.Cu") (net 16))
 (segment (start 28.31 28.81) (end 24.29 28.81) (width 0.5) (layer "F.Cu") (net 2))
 (segment (start 29.31 19.57375) (end 29.31 27.81) (width 0.5) (layer "F.Cu") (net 2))
 (segment (start 30.95625 18.57375) (end 30.31 18.57375) (width 0.5) (layer "F.Cu") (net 2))
 (arc (start 30.31 18.57375) (mid 29.602893 18.866643) (end 29.31 19.57375) (width 0.5) (layer "F.Cu") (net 2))
 (arc (start 28.31 28.81) (mid 29.017107 28.517107) (end 29.31 27.81) (width 0.5) (layer "F.Cu") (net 2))
 (segment (start 43.564213 52.033287) (end 39.84625 55.75125) (width 0.5) (layer "B.Cu") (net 17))
 (segment (start 46.19625 28.73375) (end 46.15 28.73375) (width 0.5) (layer "B.Cu") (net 17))
 (segment (start 44.15 30.73375) (end 44.15 50.619073) (width 0.5) (layer "B.Cu") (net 17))
 (arc (start 44.15 50.619073) (mid 43.997759 51.38444) (end 43.564213 52.033287) (width 0.5) (layer "B.Cu") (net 17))
 (arc (start 44.15 30.73375) (mid 44.735786 29.319536) (end 46.15 28.73375) (width 0.5) (layer "B.Cu") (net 17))
 (segment (start 29.60625 35.992177) (end 29.60625 49.40375) (width 0.5) (layer "F.Cu") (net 8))
 (segment (start 30.60625 50.40375) (end 37.30625 50.40375) (width 0.5) (layer "F.Cu") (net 8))
 (segment (start 30.95625 33.81375) (end 30.192036 34.577964) (width 0.5) (layer "F.Cu") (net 8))
 (segment (start 37.30625 50.40375) (end 37.30625 55.75125) (width 0.5) (layer "F.Cu") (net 8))
 (arc (start 29.60625 49.40375) (mid 29.899143 50.110857) (end 30.60625 50.40375) (width 0.5) (layer "F.Cu") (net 8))
 (arc (start 30.192036 34.577964) (mid 29.758491 35.22681) (end 29.60625 35.992177) (width 0.5) (layer "F.Cu") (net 8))
 (segment (start 30.95625 31.27375) (end 28.903654 33.326346) (width 0.5) (layer "F.Cu") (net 7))
 (segment (start 30.447496 51.10375) (end 34.76625 51.10375) (width 0.5) (layer "F.Cu") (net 7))
 (segment (start 34.76625 51.10375) (end 34.76625 55.75125) (width 0.5) (layer "F.Cu") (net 7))
 (segment (start 28.903654 33.326346) (end 28.903654 49.559908) (width 0.5) (layer "F.Cu") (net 7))
 (arc (start 28.903654 49.559908) (mid 29.355835 50.651569) (end 30.447496 51.10375) (width 0.5) (layer "F.Cu") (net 7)))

